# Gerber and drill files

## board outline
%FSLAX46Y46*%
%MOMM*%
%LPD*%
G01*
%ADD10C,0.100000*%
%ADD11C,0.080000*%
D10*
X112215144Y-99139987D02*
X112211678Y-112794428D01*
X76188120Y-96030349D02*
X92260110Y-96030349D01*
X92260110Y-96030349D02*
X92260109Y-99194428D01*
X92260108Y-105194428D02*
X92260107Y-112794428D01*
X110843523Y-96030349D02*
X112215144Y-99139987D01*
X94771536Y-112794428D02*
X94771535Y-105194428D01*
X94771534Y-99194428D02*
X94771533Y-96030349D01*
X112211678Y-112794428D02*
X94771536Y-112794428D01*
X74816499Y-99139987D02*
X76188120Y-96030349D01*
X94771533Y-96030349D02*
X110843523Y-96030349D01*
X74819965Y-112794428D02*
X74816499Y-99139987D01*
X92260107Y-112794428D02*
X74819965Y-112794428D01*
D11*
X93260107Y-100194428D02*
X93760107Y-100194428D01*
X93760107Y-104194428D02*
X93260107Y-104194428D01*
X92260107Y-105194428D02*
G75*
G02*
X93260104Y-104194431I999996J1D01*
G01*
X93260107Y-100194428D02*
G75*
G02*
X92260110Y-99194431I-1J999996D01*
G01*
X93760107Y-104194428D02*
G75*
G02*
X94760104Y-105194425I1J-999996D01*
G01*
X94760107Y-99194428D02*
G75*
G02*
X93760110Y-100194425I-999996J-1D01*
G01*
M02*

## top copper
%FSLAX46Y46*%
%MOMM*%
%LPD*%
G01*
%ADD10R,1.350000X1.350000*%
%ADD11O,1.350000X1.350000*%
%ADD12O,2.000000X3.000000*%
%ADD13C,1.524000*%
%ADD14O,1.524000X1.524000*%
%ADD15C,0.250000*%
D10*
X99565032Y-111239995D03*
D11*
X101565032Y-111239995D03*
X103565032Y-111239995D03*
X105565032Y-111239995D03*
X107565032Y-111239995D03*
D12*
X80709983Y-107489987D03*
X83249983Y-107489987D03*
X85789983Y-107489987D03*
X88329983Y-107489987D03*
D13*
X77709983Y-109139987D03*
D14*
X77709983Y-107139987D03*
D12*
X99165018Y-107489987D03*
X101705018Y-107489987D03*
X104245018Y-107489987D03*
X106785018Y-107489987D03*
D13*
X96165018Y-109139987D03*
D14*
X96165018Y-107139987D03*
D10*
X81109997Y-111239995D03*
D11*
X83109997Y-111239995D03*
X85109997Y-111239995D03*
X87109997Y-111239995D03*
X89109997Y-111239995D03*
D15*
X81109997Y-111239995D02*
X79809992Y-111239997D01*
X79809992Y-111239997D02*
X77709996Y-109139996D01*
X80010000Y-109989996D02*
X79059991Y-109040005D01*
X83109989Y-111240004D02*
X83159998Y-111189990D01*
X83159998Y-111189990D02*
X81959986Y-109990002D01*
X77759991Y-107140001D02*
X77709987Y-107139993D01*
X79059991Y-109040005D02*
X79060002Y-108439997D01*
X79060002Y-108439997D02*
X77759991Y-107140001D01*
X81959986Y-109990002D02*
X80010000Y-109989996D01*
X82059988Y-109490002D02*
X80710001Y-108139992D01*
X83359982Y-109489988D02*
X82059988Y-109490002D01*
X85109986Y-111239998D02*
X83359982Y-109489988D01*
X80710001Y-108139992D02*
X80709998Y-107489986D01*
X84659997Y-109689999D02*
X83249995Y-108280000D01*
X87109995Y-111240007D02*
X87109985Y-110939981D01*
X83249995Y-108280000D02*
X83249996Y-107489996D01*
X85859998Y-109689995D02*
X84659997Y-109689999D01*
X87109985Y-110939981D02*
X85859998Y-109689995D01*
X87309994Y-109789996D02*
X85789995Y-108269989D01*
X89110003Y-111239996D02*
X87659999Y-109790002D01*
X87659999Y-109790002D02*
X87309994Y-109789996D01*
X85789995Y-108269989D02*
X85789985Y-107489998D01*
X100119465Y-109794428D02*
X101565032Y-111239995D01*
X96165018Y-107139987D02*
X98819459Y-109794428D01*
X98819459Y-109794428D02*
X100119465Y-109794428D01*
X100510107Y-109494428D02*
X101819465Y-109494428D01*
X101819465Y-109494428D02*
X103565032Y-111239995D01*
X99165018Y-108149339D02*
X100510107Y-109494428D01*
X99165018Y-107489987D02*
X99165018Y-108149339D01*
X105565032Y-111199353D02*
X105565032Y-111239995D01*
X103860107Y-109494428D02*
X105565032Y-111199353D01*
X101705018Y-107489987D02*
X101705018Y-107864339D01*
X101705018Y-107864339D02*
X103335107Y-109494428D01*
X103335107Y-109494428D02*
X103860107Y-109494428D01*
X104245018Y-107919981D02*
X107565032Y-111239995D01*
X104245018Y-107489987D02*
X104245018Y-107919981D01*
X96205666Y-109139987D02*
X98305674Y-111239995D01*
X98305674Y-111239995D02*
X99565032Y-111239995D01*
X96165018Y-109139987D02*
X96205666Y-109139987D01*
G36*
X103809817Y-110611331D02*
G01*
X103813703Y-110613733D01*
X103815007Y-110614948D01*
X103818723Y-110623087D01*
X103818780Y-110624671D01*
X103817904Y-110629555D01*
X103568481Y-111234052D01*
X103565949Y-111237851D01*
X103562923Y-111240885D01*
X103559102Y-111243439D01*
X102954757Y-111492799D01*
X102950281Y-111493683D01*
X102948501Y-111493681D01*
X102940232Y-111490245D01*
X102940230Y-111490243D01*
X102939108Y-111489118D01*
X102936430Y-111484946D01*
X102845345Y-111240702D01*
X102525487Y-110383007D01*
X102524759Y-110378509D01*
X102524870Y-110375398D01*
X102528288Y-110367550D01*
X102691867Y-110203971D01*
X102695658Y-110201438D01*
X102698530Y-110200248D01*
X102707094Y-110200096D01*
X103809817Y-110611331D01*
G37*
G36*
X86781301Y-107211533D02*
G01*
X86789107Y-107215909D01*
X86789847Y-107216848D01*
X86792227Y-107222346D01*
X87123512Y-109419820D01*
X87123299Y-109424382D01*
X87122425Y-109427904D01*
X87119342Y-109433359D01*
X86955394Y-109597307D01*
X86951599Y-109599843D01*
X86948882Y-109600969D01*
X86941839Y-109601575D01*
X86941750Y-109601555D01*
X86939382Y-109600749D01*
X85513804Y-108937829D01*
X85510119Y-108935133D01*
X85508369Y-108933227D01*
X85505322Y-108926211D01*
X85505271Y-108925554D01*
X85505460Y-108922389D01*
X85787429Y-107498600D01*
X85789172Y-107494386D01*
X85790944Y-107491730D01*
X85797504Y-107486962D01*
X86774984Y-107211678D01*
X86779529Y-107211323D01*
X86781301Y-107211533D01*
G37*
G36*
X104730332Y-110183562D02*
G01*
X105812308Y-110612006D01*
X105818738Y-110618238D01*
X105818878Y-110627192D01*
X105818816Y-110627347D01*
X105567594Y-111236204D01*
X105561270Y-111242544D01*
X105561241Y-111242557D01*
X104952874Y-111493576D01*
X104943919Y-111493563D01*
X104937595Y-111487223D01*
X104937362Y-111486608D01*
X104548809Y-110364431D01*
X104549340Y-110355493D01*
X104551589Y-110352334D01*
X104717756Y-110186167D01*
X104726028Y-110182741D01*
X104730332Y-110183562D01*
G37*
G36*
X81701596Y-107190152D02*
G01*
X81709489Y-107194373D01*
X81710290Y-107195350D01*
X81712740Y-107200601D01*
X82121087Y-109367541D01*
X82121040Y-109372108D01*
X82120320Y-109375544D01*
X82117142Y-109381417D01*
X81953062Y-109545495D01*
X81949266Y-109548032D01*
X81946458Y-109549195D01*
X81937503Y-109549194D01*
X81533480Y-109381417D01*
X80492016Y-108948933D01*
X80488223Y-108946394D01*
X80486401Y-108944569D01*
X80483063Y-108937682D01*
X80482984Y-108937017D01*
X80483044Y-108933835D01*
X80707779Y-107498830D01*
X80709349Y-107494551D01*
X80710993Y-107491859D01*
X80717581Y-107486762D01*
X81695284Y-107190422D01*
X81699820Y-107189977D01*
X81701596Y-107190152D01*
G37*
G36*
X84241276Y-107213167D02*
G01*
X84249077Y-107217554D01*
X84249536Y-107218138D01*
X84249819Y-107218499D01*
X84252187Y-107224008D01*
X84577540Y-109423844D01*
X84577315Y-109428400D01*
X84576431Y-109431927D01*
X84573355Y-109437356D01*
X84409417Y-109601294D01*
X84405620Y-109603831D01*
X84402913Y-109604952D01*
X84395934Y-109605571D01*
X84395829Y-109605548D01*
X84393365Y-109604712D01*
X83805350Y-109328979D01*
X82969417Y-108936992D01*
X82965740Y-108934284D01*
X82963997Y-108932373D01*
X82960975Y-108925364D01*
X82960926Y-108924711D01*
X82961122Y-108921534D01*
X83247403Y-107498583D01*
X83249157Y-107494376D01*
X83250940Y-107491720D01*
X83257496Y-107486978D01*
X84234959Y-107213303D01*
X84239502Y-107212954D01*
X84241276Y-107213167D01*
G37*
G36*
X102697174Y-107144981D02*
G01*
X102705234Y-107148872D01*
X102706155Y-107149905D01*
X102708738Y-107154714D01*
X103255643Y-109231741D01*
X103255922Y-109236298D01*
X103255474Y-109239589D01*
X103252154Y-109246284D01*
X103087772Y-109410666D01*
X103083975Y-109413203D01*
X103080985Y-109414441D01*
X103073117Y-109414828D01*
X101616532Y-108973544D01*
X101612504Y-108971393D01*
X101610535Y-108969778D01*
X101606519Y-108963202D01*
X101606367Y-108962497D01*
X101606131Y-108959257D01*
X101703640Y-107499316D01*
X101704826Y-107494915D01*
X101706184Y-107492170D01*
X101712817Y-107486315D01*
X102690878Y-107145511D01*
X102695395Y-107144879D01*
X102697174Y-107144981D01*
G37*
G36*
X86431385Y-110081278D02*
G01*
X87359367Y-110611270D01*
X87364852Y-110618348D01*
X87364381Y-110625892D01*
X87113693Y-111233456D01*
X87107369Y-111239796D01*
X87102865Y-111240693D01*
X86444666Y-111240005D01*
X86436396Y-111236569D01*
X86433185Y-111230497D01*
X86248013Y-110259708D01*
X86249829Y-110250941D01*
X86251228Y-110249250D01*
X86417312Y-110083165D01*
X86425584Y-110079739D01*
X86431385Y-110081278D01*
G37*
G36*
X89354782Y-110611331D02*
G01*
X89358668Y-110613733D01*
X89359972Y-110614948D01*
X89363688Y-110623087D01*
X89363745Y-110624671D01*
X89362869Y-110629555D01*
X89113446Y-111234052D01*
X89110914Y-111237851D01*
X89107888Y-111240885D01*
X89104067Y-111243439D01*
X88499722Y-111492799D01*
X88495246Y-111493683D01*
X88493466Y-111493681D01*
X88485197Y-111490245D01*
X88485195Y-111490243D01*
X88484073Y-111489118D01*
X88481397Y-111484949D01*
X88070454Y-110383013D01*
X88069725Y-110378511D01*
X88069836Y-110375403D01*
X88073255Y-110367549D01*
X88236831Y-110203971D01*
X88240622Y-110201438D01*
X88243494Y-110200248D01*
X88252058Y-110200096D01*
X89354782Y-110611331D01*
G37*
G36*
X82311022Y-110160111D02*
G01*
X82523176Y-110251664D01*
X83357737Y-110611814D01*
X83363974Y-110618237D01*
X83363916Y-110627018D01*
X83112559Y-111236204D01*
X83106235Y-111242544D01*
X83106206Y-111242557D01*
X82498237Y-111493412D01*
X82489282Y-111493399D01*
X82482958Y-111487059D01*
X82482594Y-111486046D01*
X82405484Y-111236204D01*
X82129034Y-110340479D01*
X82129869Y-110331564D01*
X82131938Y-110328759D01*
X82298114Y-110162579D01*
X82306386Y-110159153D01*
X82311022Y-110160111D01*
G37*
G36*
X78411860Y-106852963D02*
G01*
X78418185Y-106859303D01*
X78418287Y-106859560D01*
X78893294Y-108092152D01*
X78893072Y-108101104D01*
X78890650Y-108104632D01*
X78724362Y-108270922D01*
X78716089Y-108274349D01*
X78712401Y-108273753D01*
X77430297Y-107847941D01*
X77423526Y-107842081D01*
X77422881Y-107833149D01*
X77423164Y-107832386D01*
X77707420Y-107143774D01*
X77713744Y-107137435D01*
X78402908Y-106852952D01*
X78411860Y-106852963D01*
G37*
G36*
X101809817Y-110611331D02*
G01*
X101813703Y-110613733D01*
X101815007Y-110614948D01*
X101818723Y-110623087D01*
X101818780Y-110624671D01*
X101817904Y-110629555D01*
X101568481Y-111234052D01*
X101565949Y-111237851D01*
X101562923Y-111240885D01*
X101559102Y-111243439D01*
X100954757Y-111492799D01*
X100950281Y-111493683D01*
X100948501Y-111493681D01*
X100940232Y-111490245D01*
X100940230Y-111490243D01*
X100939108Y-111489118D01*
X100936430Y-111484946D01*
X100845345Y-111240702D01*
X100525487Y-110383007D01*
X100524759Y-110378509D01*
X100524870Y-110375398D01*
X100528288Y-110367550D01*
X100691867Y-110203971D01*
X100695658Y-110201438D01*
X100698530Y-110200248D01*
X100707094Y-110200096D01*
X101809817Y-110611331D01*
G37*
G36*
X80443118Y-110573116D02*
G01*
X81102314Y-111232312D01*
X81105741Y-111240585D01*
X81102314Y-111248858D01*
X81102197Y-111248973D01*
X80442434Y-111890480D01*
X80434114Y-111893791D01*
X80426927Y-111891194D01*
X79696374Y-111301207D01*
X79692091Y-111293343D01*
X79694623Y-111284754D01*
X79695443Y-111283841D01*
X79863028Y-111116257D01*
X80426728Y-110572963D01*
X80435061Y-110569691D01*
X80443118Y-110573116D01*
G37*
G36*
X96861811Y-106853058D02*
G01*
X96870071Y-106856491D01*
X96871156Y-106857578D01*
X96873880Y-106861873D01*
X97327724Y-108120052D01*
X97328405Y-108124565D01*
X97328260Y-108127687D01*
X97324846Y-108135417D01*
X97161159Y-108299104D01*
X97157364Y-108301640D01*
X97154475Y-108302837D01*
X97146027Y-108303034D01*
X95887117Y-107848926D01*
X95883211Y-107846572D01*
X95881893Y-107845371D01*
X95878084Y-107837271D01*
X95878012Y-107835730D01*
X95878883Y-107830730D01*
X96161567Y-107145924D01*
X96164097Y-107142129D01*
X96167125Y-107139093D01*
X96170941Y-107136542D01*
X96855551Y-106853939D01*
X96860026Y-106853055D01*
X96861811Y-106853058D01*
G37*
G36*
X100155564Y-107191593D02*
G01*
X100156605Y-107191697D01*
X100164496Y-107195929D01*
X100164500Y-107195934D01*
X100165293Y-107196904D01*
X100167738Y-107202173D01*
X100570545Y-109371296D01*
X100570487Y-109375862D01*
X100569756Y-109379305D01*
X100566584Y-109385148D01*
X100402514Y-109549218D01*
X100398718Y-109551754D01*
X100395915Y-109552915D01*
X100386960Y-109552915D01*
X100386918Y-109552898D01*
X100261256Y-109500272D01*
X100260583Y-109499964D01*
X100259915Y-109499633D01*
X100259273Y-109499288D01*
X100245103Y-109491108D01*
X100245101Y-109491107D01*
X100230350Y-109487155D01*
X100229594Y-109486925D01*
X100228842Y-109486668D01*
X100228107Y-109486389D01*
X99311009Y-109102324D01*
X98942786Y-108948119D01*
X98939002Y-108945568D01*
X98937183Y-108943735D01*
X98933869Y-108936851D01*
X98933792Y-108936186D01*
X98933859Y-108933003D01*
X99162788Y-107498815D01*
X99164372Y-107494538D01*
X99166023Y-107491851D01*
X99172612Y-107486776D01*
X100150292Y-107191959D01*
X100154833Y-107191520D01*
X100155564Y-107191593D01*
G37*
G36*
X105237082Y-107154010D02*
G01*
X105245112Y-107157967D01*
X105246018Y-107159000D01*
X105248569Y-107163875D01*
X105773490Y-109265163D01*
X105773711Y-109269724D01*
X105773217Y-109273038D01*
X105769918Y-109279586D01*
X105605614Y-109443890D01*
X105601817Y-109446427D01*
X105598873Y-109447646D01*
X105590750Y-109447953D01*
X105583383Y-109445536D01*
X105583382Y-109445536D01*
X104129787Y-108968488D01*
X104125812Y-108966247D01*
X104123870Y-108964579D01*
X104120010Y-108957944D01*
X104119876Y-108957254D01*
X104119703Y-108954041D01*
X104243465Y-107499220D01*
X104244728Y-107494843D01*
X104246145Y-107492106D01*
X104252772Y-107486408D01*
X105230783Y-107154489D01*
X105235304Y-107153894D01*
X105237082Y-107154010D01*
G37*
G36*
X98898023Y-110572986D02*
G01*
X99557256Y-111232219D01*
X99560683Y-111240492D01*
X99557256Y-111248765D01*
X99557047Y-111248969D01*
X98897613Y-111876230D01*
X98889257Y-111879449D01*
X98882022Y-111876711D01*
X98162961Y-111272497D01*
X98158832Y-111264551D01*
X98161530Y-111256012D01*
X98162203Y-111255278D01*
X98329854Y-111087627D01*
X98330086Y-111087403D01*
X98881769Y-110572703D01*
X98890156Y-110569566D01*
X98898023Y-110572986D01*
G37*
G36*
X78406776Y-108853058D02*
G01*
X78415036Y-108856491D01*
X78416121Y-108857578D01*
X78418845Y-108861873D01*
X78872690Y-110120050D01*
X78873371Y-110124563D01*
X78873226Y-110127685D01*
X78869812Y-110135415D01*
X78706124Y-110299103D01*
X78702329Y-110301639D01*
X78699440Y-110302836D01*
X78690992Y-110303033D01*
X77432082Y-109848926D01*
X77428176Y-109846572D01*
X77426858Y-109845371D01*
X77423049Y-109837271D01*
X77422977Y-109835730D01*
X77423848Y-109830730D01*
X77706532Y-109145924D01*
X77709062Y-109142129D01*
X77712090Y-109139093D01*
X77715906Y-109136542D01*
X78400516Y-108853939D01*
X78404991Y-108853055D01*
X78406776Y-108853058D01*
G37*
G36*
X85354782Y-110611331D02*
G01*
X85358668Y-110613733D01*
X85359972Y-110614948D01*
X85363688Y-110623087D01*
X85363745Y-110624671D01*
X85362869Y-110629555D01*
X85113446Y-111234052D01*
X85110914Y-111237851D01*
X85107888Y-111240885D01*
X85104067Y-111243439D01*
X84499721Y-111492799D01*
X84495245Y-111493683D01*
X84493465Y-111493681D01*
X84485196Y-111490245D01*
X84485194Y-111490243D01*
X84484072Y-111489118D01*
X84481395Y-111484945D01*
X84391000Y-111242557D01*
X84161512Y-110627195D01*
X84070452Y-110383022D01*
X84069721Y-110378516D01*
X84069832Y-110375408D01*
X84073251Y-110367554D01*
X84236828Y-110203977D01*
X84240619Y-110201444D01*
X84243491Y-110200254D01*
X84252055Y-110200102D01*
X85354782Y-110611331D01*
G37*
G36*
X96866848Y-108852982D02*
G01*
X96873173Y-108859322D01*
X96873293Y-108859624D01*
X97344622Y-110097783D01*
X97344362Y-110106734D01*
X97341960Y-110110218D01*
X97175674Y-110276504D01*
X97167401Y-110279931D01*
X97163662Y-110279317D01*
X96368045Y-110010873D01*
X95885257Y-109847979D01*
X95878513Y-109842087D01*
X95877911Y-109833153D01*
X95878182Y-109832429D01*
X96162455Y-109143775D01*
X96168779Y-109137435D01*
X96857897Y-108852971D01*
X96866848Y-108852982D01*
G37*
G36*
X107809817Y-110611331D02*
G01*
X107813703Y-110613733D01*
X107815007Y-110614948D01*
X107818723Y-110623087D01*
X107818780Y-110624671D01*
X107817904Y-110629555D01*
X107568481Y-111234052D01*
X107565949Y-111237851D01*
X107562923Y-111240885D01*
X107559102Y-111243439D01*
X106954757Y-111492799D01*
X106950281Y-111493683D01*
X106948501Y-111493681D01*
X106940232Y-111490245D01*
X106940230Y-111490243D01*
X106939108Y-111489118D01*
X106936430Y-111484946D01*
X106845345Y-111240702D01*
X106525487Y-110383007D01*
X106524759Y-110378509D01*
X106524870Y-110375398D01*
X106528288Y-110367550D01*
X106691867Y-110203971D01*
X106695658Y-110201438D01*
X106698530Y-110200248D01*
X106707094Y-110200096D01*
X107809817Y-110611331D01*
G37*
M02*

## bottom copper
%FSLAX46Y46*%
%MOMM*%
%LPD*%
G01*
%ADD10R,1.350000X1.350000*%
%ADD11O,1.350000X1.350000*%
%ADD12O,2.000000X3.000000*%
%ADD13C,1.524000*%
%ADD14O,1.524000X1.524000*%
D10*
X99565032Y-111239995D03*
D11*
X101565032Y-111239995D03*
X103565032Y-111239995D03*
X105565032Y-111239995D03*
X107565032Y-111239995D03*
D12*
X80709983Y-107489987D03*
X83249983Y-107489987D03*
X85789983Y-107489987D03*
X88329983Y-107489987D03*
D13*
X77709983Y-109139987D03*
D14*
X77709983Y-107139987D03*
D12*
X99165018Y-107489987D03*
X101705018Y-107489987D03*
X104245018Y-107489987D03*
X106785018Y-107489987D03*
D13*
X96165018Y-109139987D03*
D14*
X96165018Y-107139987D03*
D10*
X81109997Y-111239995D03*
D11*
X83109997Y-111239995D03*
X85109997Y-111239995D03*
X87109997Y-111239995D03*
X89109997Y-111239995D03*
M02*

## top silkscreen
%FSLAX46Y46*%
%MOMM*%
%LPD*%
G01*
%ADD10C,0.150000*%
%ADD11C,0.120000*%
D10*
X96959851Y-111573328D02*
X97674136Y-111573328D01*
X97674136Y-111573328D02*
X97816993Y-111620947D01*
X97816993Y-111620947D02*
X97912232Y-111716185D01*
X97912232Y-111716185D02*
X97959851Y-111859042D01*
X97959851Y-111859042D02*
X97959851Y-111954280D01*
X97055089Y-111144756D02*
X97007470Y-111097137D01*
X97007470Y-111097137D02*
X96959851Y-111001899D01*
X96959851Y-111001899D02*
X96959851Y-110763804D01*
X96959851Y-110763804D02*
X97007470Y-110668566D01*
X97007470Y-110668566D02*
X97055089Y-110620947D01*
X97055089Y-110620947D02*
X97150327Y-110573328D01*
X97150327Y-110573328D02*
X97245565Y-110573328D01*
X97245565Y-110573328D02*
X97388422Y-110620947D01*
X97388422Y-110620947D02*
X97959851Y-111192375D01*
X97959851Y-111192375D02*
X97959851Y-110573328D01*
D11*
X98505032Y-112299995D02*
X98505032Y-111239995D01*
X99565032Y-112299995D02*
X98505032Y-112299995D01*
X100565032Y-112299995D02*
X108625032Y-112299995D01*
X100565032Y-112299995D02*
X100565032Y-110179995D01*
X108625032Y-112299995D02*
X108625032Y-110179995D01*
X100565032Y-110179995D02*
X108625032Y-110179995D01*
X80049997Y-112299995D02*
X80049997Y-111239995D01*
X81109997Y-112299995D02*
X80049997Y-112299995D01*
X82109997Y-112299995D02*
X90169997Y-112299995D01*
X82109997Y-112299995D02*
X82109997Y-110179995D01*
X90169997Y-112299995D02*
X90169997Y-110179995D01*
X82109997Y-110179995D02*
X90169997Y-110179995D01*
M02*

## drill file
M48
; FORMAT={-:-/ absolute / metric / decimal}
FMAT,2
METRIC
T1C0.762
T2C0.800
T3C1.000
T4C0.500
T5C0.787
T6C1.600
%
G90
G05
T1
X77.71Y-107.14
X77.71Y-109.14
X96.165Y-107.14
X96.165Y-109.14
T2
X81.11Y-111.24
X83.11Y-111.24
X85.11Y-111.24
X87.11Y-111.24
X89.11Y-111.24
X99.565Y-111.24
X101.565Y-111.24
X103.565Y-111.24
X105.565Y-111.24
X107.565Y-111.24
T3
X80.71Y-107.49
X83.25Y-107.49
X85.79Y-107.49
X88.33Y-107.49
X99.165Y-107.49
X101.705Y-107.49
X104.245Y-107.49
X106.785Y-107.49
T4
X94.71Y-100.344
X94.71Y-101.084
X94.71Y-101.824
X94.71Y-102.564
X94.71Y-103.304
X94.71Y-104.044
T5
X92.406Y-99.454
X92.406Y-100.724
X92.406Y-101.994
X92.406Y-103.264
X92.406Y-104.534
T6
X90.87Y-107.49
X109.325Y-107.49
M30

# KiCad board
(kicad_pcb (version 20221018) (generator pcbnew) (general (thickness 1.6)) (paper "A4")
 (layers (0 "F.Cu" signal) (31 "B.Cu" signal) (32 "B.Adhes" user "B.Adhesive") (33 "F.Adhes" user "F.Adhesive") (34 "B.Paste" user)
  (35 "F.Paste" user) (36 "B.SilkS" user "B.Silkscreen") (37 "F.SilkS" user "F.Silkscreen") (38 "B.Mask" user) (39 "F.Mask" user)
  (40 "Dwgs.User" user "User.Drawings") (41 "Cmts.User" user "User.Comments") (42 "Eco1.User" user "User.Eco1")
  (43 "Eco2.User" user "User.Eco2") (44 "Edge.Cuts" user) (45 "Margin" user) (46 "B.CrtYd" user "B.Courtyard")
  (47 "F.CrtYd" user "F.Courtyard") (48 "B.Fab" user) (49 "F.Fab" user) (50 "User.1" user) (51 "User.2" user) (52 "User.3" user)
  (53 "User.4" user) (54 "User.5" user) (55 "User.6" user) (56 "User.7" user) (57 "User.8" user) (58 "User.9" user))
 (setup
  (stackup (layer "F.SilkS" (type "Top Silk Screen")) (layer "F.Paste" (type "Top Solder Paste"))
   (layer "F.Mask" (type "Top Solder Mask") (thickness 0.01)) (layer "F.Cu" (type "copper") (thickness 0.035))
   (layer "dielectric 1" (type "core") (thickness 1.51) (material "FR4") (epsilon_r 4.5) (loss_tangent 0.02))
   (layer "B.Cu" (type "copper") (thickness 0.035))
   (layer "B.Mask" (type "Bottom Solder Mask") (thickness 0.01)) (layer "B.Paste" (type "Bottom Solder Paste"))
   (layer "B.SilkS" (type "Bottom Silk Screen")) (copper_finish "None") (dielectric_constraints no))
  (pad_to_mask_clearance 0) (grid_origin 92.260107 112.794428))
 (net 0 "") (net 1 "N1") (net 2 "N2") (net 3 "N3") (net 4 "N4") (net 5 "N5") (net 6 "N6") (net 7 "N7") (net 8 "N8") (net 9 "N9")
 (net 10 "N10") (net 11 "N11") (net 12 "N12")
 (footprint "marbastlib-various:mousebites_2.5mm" (layer "F.Cu") (at 94.760107 102.194428)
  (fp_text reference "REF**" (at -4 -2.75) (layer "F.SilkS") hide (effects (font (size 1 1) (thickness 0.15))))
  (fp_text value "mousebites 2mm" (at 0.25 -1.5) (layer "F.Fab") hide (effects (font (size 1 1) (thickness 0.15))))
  (fp_line (start -1.5 -2) (end -1 -2) (stroke (width 0.08) (type solid)) (layer "Edge.Cuts"))
  (fp_line (start -1 2) (end -1.5 2) (stroke (width 0.08) (type solid)) (layer "Edge.Cuts"))
  (fp_arc (start -2.5 3) (mid -2.207108 2.292895) (end -1.500003 2.000003) (stroke (width 0.08) (type solid)) (layer "Edge.Cuts"))
  (fp_arc (start -1.5 -2) (mid -2.207105 -2.292892) (end -2.499997 -2.999997) (stroke (width 0.08) (type solid)) (layer "Edge.Cuts"))
  (fp_arc (start -1 2) (mid -0.292895 2.292892) (end -0.000003 2.999997) (stroke (width 0.08) (type solid)) (layer "Edge.Cuts"))
  (fp_arc (start 0 -3) (mid -0.292892 -2.292895) (end -0.999997 -2.000003) (stroke (width 0.08) (type solid)) (layer "Edge.Cuts"))
  (pad "" np_thru_hole circle (at -0.05 -1.85) (size 0.5 0.5) (drill 0.5) (layers F&B.Cu *.Mask))
  (pad "" np_thru_hole circle (at -0.05 -1.11) (size 0.5 0.5) (drill 0.5) (layers F&B.Cu *.Mask))
  (pad "" np_thru_hole circle (at -0.05 -0.37) (size 0.5 0.5) (drill 0.5) (layers F&B.Cu *.Mask))
  (pad "" np_thru_hole circle (at -0.05 0.37) (size 0.5 0.5) (drill 0.5) (layers F&B.Cu *.Mask))
  (pad "" np_thru_hole circle (at -0.05 1.11) (size 0.5 0.5) (drill 0.5) (layers F&B.Cu *.Mask))
  (pad "" np_thru_hole circle (at -0.05 1.85) (size 0.5 0.5) (drill 0.5) (layers F&B.Cu *.Mask)))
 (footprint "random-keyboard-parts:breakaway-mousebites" (layer "F.Cu") (at 92.660107 101.994428 90)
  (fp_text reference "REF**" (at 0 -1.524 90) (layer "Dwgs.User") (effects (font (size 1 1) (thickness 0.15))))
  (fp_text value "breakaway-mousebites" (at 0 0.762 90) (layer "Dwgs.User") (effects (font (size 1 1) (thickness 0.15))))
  (pad "" np_thru_hole circle (at -2.54 -0.254 90) (size 0.7874 0.7874) (drill 0.7874) (layers *.Cu *.Mask))
  (pad "" np_thru_hole circle (at -1.27 -0.254 90) (size 0.7874 0.7874) (drill 0.7874) (layers *.Cu *.Mask))
  (pad "" np_thru_hole circle (at 0 -0.254 90) (size 0.7874 0.7874) (drill 0.7874) (layers *.Cu *.Mask))
  (pad "" np_thru_hole circle (at 1.27 -0.254 90) (size 0.7874 0.7874) (drill 0.7874) (layers *.Cu *.Mask))
  (pad "" np_thru_hole circle (at 2.54 -0.254 90) (size 0.7874 0.7874) (drill 0.7874) (layers *.Cu *.Mask)))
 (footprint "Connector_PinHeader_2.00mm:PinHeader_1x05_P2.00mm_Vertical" (layer "F.Cu") (at 99.565032 111.239995 90)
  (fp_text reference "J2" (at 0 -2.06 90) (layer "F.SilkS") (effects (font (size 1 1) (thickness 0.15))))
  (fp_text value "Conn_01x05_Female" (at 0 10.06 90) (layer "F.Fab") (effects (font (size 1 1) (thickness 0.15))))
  (fp_line (start -1.06 -1.06) (end 0 -1.06) (stroke (width 0.12) (type solid)) (layer "F.SilkS"))
  (fp_line (start -1.06 0) (end -1.06 -1.06) (stroke (width 0.12) (type solid)) (layer "F.SilkS"))
  (fp_line (start -1.06 1) (end -1.06 9.06) (stroke (width 0.12) (type solid)) (layer "F.SilkS"))
  (fp_line (start -1.06 1) (end 1.06 1) (stroke (width 0.12) (type solid)) (layer "F.SilkS"))
  (fp_line (start -1.06 9.06) (end 1.06 9.06) (stroke (width 0.12) (type solid)) (layer "F.SilkS"))
  (fp_line (start 1.06 1) (end 1.06 9.06) (stroke (width 0.12) (type solid)) (layer "F.SilkS"))
  (pad "1" thru_hole rect (at 0 0 90) (size 1.35 1.35) (drill 0.8) (layers *.Cu *.Mask) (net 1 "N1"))
  (pad "2" thru_hole oval (at 0 2 90) (size 1.35 1.35) (drill 0.8) (layers *.Cu *.Mask) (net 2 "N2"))
  (pad "3" thru_hole oval (at 0 4 90) (size 1.35 1.35) (drill 0.8) (layers *.Cu *.Mask) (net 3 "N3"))
  (pad "4" thru_hole oval (at 0 6 90) (size 1.35 1.35) (drill 0.8) (layers *.Cu *.Mask) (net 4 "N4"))
  (pad "5" thru_hole oval (at 0 8 90) (size 1.35 1.35) (drill 0.8) (layers *.Cu *.Mask) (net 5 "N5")))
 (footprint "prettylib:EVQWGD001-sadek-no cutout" (layer "F.Cu") (at 84.659983 101.639987 180)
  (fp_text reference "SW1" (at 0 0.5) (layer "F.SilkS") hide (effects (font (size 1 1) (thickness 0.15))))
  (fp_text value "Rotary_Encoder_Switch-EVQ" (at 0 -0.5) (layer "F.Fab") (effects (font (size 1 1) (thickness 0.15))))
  (pad "" np_thru_hole circle (at -6.21 -5.85 180) (size 1.6 1.6) (drill 1.6) (layers *.Cu))
  (pad "A" thru_hole oval (at 3.95 -5.85 180) (size 2 3) (drill 1) (layers *.Cu *.Mask) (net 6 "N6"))
  (pad "B" thru_hole oval (at 1.41 -5.85 180) (size 2 3) (drill 1) (layers *.Cu *.Mask) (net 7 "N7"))
  (pad "C" thru_hole oval (at -1.13 -5.85 180) (size 2 3) (drill 1) (layers *.Cu *.Mask) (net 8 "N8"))
  (pad "NC" thru_hole oval (at -3.67 -5.85 180) (size 2 3) (drill 1) (layers *.Cu *.Mask) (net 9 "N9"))
  (pad "S1" thru_hole circle (at 6.95 -7.5 180) (size 1.524 1.524) (drill 0.762) (layers *.Cu *.Mask) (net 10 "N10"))
  (pad "S2" thru_hole oval (at 6.95 -5.5 180) (size 1.524 1.524) (drill 0.762) (layers *.Cu *.Mask) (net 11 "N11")))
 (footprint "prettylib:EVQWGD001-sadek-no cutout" (layer "F.Cu") (at 103.115018 101.639987 180)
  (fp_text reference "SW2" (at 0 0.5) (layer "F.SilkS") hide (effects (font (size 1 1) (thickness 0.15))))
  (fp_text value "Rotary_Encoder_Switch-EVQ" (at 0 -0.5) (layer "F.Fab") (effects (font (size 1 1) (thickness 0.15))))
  (pad "" np_thru_hole circle (at -6.21 -5.85 180) (size 1.6 1.6) (drill 1.6) (layers *.Cu))
  (pad "A" thru_hole oval (at 3.95 -5.85 180) (size 2 3) (drill 1) (layers *.Cu *.Mask) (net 3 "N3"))
  (pad "B" thru_hole oval (at 1.41 -5.85 180) (size 2 3) (drill 1) (layers *.Cu *.Mask) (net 4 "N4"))
  (pad "C" thru_hole oval (at -1.13 -5.85 180) (size 2 3) (drill 1) (layers *.Cu *.Mask) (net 5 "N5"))
  (pad "NC" thru_hole oval (at -3.67 -5.85 180) (size 2 3) (drill 1) (layers *.Cu *.Mask) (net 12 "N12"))
  (pad "S1" thru_hole circle (at 6.95 -7.5 180) (size 1.524 1.524) (drill 0.762) (layers *.Cu *.Mask) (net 1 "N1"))
  (pad "S2" thru_hole oval (at 6.95 -5.5 180) (size 1.524 1.524) (drill 0.762) (layers *.Cu *.Mask) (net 2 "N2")))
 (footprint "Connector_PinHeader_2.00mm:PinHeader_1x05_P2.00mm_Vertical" (layer "F.Cu") (at 81.109997 111.239995 90)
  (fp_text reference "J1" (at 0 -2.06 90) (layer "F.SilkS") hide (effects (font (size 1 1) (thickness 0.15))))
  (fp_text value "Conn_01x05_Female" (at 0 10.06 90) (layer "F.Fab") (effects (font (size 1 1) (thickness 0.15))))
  (fp_line (start -1.06 -1.06) (end 0 -1.06) (stroke (width 0.12) (type solid)) (layer "F.SilkS"))
  (fp_line (start -1.06 0) (end -1.06 -1.06) (stroke (width 0.12) (type solid)) (layer "F.SilkS"))
  (fp_line (start -1.06 1) (end -1.06 9.06) (stroke (width 0.12) (type solid)) (layer "F.SilkS"))
  (fp_line (start -1.06 1) (end 1.06 1) (stroke (width 0.12) (type solid)) (layer "F.SilkS"))
  (fp_line (start -1.06 9.06) (end 1.06 9.06) (stroke (width 0.12) (type solid)) (layer "F.SilkS"))
  (fp_line (start 1.06 1) (end 1.06 9.06) (stroke (width 0.12) (type solid)) (layer "F.SilkS"))
  (pad "1" thru_hole rect (at 0 0 90) (size 1.35 1.35) (drill 0.8) (layers *.Cu *.Mask) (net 10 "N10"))
  (pad "2" thru_hole oval (at 0 2 90) (size 1.35 1.35) (drill 0.8) (layers *.Cu *.Mask) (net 11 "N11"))
  (pad "3" thru_hole oval (at 0 4 90) (size 1.35 1.35) (drill 0.8) (layers *.Cu *.Mask) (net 6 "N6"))
  (pad "4" thru_hole oval (at 0 6 90) (size 1.35 1.35) (drill 0.8) (layers *.Cu *.Mask) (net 7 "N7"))
  (pad "5" thru_hole oval (at 0 8 90) (size 1.35 1.35) (drill 0.8) (layers *.Cu *.Mask) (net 8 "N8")))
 (gr_line (start 112.215144 99.139987) (end 112.211678 112.794428) (stroke (width 0.1) (type solid)) (layer "Edge.Cuts"))
 (gr_line (start 76.18812 96.030349) (end 92.26011 96.030349) (stroke (width 0.1) (type solid)) (layer "Edge.Cuts"))
 (gr_line (start 92.26011 96.030349) (end 92.260109 99.194428) (stroke (width 0.1) (type solid)) (layer "Edge.Cuts"))
 (gr_line (start 92.260108 105.194428) (end 92.260107 112.794428) (stroke (width 0.1) (type solid)) (layer "Edge.Cuts"))
 (gr_line (start 110.843523 96.030349) (end 112.215144 99.139987) (stroke (width 0.1) (type solid)) (layer "Edge.Cuts"))
 (gr_line (start 94.771536 112.794428) (end 94.771535 105.194428) (stroke (width 0.1) (type solid)) (layer "Edge.Cuts"))
 (gr_line (start 94.771534 99.194428) (end 94.771533 96.030349) (stroke (width 0.1) (type solid)) (layer "Edge.Cuts"))
 (gr_line (start 112.211678 112.794428) (end 94.771536 112.794428) (stroke (width 0.1) (type solid)) (layer "Edge.Cuts"))
 (gr_line (start 74.816499 99.139987) (end 76.18812 96.030349) (stroke (width 0.1) (type solid)) (layer "Edge.Cuts"))
 (gr_line (start 94.771533 96.030349) (end 110.843523 96.030349) (stroke (width 0.1) (type solid)) (layer "Edge.Cuts"))
 (gr_line (start 74.819965 112.794428) (end 74.816499 99.139987) (stroke (width 0.1) (type solid)) (layer "Edge.Cuts"))
 (gr_line (start 92.260107 112.794428) (end 74.819965 112.794428) (stroke (width 0.1) (type solid)) (layer "Edge.Cuts"))
 (segment (start 81.109997 111.239995) (end 79.809992 111.239997) (width 0.25) (layer "F.Cu") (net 10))
 (segment (start 79.809992 111.239997) (end 77.709996 109.139996) (width 0.25) (layer "F.Cu") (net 10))
 (segment (start 80.01 109.989996) (end 79.059991 109.040005) (width 0.25) (layer "F.Cu") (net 11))
 (segment (start 83.109989 111.240004) (end 83.159998 111.18999) (width 0.25) (layer "F.Cu") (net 11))
 (segment (start 83.159998 111.18999) (end 81.959986 109.990002) (width 0.25) (layer "F.Cu") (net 11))
 (segment (start 77.759991 107.140001) (end 77.709987 107.139993) (width 0.25) (layer "F.Cu") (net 11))
 (segment (start 79.059991 109.040005) (end 79.060002 108.439997) (width 0.25) (layer "F.Cu") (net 11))
 (segment (start 79.060002 108.439997) (end 77.759991 107.140001) (width 0.25) (layer "F.Cu") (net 11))
 (segment (start 81.959986 109.990002) (end 80.01 109.989996) (width 0.25) (layer "F.Cu") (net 11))
 (segment (start 82.059988 109.490002) (end 80.710001 108.139992) (width 0.25) (layer "F.Cu") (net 6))
 (segment (start 83.359982 109.489988) (end 82.059988 109.490002) (width 0.25) (layer "F.Cu") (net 6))
 (segment (start 85.109986 111.239998) (end 83.359982 109.489988) (width 0.25) (layer "F.Cu") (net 6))
 (segment (start 80.710001 108.139992) (end 80.709998 107.489986) (width 0.25) (layer "F.Cu") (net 6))
 (segment (start 84.659997 109.689999) (end 83.249995 108.28) (width 0.25) (layer "F.Cu") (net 7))
 (segment (start 87.109995 111.240007) (end 87.109985 110.939981) (width 0.25) (layer "F.Cu") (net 7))
 (segment (start 83.249995 108.28) (end 83.249996 107.489996) (width 0.25) (layer "F.Cu") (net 7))
 (segment (start 85.859998 109.689995) (end 84.659997 109.689999) (width 0.25) (layer "F.Cu") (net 7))
 (segment (start 87.109985 110.939981) (end 85.859998 109.689995) (width 0.25) (layer "F.Cu") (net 7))
 (segment (start 87.309994 109.789996) (end 85.789995 108.269989) (width 0.25) (layer "F.Cu") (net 8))
 (segment (start 89.110003 111.239996) (end 87.659999 109.790002) (width 0.25) (layer "F.Cu") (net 8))
 (segment (start 87.659999 109.790002) (end 87.309994 109.789996) (width 0.25) (layer "F.Cu") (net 8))
 (segment (start 85.789995 108.269989) (end 85.789985 107.489998) (width 0.25) (layer "F.Cu") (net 8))
 (segment (start 100.119465 109.794428) (end 101.565032 111.239995) (width 0.25) (layer "F.Cu") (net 2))
 (segment (start 96.165018 107.139987) (end 98.819459 109.794428) (width 0.25) (layer "F.Cu") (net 2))
 (segment (start 98.819459 109.794428) (end 100.119465 109.794428) (width 0.25) (layer "F.Cu") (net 2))
 (segment (start 100.510107 109.494428) (end 101.819465 109.494428) (width 0.25) (layer "F.Cu") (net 3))
 (segment (start 101.819465 109.494428) (end 103.565032 111.239995) (width 0.25) (layer "F.Cu") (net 3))
 (segment (start 99.165018 108.149339) (end 100.510107 109.494428) (width 0.25) (layer "F.Cu") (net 3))
 (segment (start 99.165018 107.489987) (end 99.165018 108.149339) (width 0.25) (layer "F.Cu") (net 3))
 (segment (start 105.565032 111.199353) (end 105.565032 111.239995) (width 0.25) (layer "F.Cu") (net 4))
 (segment (start 103.860107 109.494428) (end 105.565032 111.199353) (width 0.25) (layer "F.Cu") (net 4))
 (segment (start 101.705018 107.489987) (end 101.705018 107.864339) (width 0.25) (layer "F.Cu") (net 4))
 (segment (start 101.705018 107.864339) (end 103.335107 109.494428) (width 0.25) (layer "F.Cu") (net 4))
 (segment (start 103.335107 109.494428) (end 103.860107 109.494428) (width 0.25) (layer "F.Cu") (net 4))
 (segment (start 104.245018 107.919981) (end 107.565032 111.239995) (width 0.25) (layer "F.Cu") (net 5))
 (segment (start 104.245018 107.489987) (end 104.245018 107.919981) (width 0.25) (layer "F.Cu") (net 5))
 (segment (start 96.205666 109.139987) (end 98.305674 111.239995) (width 0.25) (layer "F.Cu") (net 1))
 (segment (start 98.305674 111.239995) (end 99.565032 111.239995) (width 0.25) (layer "F.Cu") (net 1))
 (segment (start 96.165018 109.139987) (end 96.205666 109.139987) (width 0.25) (layer "F.Cu") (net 1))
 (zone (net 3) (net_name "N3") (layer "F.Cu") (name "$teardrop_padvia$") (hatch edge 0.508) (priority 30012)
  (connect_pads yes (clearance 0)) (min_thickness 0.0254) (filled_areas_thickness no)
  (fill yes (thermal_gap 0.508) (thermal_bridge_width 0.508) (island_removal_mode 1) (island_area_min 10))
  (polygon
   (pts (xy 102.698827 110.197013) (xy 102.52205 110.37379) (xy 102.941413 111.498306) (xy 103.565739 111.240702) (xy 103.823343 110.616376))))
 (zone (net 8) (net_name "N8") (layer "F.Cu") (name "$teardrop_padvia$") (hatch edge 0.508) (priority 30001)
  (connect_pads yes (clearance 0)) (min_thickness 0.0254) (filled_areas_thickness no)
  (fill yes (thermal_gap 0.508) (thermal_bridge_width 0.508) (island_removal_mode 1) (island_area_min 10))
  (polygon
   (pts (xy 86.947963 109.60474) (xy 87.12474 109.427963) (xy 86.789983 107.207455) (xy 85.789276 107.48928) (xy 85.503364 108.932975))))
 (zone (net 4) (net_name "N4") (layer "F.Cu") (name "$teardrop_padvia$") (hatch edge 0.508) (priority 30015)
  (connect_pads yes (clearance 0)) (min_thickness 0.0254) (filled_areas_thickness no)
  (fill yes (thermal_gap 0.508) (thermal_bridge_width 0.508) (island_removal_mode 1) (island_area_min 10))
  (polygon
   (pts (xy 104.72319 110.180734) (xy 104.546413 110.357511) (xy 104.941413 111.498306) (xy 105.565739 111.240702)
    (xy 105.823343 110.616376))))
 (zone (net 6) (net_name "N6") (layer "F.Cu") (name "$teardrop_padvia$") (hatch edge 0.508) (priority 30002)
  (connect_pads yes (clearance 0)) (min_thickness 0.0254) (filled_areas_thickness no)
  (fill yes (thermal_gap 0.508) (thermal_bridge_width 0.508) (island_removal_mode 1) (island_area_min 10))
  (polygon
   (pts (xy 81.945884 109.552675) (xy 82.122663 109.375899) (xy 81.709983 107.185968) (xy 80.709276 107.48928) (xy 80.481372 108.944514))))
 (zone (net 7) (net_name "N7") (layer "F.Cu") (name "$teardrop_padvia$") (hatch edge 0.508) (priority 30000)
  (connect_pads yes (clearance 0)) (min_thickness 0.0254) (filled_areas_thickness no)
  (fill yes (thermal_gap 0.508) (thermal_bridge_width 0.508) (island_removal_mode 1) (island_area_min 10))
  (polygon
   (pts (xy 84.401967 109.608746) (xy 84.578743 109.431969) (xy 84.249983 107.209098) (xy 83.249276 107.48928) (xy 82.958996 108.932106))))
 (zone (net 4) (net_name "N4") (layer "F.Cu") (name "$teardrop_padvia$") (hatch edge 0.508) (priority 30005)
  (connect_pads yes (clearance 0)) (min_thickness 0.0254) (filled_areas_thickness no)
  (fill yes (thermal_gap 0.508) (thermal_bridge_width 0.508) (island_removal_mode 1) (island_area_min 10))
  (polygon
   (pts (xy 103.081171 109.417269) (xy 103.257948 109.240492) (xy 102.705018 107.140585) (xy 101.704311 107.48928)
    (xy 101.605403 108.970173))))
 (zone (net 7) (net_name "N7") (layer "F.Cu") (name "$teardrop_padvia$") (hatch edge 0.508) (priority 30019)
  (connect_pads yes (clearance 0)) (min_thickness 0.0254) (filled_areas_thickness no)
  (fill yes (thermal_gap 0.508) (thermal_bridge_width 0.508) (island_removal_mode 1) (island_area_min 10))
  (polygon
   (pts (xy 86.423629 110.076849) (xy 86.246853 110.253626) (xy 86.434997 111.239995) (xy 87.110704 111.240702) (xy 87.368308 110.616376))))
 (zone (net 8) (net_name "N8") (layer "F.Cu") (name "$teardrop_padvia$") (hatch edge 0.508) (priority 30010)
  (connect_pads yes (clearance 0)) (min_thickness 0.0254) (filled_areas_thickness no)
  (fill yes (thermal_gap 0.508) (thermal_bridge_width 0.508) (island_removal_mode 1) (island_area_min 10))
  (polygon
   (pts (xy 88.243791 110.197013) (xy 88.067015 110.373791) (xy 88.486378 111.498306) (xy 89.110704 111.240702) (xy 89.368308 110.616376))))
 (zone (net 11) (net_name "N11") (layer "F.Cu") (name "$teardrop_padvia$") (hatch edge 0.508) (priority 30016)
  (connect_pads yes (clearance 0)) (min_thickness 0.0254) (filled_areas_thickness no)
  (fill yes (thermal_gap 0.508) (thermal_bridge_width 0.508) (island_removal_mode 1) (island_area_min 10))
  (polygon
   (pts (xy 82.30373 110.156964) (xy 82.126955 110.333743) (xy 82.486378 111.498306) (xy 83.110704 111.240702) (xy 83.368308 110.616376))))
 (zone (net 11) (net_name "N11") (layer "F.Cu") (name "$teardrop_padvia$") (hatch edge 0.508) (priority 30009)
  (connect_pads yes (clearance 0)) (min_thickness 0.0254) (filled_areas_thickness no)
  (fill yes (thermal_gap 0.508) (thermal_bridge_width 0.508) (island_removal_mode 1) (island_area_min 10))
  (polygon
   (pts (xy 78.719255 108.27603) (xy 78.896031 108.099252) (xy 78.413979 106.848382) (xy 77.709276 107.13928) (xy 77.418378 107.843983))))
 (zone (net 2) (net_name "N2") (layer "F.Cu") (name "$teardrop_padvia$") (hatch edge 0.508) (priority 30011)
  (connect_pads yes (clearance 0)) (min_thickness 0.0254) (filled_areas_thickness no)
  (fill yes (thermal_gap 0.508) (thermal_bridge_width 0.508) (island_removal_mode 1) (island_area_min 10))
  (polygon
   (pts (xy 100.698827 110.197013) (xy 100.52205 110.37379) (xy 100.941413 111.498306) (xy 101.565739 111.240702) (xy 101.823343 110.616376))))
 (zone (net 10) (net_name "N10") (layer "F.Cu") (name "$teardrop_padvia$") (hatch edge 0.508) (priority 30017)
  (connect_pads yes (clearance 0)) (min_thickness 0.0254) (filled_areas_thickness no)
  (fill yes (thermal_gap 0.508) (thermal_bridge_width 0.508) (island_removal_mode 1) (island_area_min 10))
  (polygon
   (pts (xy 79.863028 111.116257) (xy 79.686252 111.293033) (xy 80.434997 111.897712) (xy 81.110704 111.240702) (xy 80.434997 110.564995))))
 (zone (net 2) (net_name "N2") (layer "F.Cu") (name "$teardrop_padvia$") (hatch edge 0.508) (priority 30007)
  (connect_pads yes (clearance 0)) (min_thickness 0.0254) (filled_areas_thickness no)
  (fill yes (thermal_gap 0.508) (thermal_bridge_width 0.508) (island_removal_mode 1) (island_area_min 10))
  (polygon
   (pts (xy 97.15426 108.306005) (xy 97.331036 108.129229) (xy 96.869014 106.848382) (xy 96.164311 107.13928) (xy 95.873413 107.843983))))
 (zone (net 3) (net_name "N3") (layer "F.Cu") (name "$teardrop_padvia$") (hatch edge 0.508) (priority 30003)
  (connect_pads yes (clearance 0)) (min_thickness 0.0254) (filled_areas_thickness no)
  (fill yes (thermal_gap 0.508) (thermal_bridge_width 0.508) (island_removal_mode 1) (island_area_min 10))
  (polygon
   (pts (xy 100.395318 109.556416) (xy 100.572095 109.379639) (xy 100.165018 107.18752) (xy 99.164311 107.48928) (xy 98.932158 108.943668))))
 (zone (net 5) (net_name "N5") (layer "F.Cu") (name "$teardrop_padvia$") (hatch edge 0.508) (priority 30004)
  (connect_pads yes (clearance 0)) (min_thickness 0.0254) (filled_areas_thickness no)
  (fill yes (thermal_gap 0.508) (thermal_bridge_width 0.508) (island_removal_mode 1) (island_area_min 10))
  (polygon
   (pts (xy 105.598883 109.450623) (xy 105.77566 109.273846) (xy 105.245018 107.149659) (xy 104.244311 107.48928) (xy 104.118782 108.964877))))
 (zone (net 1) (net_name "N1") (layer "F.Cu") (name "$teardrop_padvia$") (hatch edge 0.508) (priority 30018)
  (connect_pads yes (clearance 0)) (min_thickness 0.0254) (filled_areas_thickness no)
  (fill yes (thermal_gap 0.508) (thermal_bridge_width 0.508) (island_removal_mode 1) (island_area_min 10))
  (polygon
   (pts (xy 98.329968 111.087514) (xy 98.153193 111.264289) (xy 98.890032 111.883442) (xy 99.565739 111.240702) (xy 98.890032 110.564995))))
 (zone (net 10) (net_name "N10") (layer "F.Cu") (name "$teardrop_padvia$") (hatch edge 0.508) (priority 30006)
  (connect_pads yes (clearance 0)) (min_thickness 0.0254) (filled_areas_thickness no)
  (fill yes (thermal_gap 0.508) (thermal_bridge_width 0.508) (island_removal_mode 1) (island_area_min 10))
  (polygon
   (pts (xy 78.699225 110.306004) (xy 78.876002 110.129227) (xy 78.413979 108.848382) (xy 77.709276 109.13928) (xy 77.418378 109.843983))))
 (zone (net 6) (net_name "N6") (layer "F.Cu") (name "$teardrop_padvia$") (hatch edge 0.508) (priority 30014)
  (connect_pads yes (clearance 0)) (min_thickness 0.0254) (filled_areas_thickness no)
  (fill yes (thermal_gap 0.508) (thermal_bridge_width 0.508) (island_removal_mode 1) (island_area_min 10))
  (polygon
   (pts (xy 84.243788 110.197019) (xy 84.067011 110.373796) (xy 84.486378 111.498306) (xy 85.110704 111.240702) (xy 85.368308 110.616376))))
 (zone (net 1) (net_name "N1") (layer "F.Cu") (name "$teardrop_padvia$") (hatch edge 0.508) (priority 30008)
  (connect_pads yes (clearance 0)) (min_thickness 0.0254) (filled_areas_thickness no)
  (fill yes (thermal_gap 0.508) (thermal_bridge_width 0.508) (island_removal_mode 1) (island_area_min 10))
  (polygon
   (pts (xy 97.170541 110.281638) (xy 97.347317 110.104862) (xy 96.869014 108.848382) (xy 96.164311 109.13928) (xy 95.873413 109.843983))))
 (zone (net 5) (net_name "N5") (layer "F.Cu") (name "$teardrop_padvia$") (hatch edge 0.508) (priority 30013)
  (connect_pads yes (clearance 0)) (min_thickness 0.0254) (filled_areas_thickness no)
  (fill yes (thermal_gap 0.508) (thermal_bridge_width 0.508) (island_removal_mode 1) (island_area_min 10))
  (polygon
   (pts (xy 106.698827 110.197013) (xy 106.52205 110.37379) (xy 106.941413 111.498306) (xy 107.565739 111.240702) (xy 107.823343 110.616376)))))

